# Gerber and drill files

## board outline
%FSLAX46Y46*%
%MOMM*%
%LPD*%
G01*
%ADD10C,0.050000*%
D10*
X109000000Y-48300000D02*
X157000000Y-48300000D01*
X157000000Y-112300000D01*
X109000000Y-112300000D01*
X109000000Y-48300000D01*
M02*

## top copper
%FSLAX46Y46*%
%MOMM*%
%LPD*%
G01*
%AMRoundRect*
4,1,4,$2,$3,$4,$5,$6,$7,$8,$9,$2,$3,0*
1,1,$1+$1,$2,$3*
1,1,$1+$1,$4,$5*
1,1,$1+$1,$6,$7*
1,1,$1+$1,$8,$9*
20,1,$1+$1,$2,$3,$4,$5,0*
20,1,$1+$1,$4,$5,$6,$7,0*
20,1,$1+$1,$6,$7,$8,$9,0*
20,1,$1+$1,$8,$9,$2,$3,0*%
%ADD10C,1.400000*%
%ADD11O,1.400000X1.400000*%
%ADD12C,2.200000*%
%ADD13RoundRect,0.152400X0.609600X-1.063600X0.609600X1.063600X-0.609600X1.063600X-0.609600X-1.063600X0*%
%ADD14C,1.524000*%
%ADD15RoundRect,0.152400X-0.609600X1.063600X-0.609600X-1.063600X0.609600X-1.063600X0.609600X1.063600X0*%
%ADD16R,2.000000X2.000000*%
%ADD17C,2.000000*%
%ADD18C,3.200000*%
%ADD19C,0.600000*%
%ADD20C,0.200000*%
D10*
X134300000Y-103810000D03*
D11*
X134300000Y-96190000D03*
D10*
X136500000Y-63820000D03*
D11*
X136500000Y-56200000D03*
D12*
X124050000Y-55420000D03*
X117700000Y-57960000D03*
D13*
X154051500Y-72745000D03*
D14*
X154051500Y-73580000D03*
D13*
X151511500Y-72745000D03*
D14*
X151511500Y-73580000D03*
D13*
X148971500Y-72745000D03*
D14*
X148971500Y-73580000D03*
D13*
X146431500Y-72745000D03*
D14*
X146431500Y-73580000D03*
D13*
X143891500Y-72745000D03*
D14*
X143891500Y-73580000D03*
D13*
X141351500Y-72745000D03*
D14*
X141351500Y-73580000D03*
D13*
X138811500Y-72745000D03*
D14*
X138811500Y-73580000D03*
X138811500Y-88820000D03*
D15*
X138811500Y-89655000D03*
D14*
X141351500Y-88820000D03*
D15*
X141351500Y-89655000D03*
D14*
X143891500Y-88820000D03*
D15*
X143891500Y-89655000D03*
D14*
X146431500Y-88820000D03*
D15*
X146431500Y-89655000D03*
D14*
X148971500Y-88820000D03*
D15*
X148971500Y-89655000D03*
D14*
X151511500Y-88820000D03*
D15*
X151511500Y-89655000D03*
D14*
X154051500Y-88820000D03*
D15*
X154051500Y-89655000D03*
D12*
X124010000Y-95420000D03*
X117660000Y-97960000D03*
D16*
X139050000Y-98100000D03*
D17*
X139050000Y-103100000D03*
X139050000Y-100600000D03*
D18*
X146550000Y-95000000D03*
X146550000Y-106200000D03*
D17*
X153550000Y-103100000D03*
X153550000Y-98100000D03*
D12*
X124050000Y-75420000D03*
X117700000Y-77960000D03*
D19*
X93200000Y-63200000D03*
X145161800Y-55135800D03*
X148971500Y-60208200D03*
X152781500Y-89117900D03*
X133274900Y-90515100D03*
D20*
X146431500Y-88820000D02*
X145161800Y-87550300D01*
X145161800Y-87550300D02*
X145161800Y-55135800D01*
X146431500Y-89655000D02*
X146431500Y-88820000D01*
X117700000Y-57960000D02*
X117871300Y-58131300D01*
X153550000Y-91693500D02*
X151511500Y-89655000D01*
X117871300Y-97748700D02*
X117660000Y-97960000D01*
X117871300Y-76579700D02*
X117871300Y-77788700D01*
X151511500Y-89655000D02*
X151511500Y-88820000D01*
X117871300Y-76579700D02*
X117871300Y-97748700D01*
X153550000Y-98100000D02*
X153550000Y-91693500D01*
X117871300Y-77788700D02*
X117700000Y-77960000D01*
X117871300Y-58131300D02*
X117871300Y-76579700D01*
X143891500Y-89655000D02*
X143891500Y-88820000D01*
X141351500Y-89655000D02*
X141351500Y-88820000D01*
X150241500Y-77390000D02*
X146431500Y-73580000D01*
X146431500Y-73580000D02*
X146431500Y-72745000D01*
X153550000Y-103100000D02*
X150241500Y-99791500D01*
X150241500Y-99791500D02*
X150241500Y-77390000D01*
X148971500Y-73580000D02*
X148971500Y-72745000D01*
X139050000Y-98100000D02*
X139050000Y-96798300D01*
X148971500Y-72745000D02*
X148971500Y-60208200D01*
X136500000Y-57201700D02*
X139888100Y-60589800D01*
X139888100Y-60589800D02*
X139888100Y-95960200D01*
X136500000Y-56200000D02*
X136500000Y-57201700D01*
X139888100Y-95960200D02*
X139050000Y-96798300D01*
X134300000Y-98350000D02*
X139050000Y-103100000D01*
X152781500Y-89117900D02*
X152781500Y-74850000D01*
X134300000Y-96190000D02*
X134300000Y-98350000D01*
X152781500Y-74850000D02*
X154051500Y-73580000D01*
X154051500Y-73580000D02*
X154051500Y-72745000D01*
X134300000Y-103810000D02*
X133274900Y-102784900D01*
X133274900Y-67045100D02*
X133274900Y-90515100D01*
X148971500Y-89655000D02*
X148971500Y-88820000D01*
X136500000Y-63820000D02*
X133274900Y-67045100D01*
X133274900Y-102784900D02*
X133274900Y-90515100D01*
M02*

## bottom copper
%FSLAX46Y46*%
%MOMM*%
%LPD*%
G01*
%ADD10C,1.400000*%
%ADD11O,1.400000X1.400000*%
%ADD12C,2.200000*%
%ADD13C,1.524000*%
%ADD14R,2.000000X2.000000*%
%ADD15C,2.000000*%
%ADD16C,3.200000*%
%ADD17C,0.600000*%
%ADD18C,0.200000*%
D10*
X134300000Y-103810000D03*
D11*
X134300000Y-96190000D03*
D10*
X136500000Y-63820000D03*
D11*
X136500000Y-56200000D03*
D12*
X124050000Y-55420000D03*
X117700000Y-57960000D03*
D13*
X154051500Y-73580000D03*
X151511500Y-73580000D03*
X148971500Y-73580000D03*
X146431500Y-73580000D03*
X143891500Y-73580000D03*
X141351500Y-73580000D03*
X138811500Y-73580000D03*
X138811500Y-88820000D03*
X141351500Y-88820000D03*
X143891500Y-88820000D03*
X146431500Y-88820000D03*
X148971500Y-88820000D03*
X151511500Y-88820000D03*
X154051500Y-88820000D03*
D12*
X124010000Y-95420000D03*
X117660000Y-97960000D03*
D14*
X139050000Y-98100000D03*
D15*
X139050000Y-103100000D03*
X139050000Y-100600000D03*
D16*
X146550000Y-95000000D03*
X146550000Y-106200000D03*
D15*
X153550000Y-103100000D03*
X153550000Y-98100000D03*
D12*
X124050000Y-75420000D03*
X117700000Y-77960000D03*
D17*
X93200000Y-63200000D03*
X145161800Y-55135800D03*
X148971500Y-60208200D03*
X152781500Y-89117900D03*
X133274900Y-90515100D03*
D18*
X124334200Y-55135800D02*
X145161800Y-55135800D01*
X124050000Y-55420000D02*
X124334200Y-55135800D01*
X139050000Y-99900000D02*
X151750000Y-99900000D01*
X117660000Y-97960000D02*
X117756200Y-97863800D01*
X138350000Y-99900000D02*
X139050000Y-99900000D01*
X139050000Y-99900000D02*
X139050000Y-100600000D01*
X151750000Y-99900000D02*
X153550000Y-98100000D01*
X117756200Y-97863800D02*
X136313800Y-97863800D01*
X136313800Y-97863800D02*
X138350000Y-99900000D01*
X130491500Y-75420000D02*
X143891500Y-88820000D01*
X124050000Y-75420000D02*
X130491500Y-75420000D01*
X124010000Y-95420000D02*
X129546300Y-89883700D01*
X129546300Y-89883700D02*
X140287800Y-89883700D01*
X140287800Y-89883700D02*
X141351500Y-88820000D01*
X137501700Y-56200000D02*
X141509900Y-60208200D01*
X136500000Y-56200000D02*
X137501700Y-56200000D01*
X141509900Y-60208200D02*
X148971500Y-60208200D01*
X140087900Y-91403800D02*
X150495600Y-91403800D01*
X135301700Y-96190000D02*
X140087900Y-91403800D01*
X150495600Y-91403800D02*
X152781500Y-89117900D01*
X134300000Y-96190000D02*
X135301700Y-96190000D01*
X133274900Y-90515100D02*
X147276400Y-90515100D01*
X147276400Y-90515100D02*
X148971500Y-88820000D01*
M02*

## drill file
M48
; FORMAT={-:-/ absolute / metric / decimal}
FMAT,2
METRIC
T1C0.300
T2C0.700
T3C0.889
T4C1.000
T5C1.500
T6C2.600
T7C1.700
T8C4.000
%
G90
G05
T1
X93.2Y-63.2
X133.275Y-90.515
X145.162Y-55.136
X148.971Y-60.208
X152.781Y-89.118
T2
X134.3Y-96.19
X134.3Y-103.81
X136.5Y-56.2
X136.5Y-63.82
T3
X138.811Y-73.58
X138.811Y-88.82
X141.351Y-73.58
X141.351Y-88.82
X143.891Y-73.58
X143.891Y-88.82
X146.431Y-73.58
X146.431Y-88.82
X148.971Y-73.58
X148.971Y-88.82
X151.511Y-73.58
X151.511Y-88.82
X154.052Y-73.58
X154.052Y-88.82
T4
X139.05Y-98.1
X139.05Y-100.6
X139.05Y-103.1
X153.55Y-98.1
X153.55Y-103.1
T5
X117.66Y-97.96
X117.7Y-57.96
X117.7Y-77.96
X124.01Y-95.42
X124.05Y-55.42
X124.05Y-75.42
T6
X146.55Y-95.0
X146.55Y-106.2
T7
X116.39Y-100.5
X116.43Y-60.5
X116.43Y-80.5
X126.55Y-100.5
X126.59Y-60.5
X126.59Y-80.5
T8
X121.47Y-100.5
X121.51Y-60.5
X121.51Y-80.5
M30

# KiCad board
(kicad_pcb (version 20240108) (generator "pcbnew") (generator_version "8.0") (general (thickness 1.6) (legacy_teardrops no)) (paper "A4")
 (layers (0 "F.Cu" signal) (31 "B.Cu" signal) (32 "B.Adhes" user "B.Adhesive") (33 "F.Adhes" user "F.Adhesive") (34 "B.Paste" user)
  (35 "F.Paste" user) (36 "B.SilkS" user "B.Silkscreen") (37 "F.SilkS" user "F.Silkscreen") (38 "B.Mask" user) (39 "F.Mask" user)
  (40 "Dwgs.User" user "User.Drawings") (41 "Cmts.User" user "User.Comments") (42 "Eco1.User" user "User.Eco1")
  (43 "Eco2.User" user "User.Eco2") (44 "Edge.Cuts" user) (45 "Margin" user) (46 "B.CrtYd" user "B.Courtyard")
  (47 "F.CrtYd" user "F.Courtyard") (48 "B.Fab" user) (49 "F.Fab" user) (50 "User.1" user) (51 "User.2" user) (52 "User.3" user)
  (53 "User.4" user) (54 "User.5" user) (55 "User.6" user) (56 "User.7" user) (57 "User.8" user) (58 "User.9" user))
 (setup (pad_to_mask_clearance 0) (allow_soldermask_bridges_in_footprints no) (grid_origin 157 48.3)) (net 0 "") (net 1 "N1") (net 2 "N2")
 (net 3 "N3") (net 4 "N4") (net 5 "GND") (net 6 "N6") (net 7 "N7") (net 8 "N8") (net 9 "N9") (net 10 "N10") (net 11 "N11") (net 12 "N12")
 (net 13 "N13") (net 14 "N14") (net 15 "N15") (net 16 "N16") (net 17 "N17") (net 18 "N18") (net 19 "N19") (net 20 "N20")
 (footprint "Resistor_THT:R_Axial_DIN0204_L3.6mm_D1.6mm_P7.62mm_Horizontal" (layer "F.Cu") (at 134.3 103.81 90)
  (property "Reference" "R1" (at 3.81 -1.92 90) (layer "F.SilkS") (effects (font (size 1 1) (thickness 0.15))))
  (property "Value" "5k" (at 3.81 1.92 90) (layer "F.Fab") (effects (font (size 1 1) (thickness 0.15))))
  (pad "1" thru_hole circle (at 0 0 90) (size 1.4 1.4) (drill 0.7) (layers "*.Cu" "*.Mask") (remove_unused_layers no) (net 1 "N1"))
  (pad "2" thru_hole oval (at 7.62 0 90) (size 1.4 1.4) (drill 0.7) (layers "*.Cu" "*.Mask") (remove_unused_layers no) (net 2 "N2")))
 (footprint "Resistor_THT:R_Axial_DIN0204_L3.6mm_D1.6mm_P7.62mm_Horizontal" (layer "F.Cu") (at 136.5 63.82 90)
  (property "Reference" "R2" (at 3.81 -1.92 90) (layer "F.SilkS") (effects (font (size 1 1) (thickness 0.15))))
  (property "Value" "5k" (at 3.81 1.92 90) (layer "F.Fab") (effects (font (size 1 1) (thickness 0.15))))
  (pad "1" thru_hole circle (at 0 0 90) (size 1.4 1.4) (drill 0.7) (layers "*.Cu" "*.Mask") (remove_unused_layers no) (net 1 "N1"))
  (pad "2" thru_hole oval (at 7.62 0 90) (size 1.4 1.4) (drill 0.7) (layers "*.Cu" "*.Mask") (remove_unused_layers no) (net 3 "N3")))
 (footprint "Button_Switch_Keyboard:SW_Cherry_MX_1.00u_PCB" (layer "F.Cu") (at 124.05 55.42)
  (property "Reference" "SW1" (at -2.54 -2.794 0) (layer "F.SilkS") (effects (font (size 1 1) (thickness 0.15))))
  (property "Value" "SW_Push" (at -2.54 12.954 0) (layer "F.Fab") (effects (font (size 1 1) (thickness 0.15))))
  (pad "" np_thru_hole circle (at -7.62 5.08) (size 1.7 1.7) (drill 1.7) (layers "*.Cu" "*.Mask"))
  (pad "" np_thru_hole circle (at -2.54 5.08) (size 4 4) (drill 4) (layers "*.Cu" "*.Mask"))
  (pad "" np_thru_hole circle (at 2.54 5.08) (size 1.7 1.7) (drill 1.7) (layers "*.Cu" "*.Mask"))
  (pad "1" thru_hole circle (at 0 0) (size 2.2 2.2) (drill 1.5) (layers "*.Cu" "*.Mask") (remove_unused_layers no) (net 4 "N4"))
  (pad "2" thru_hole circle (at -6.35 2.54) (size 2.2 2.2) (drill 1.5) (layers "*.Cu" "*.Mask") (remove_unused_layers no) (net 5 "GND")))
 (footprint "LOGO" (layer "F.Cu") (at 148.920677 59.275013 -90)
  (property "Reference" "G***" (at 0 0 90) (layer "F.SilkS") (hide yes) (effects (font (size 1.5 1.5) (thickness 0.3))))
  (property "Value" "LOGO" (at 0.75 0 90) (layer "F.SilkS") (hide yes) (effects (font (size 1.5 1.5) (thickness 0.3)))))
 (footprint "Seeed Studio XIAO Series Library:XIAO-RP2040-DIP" (layer "F.Cu") (at 146.4315 81.2 -90)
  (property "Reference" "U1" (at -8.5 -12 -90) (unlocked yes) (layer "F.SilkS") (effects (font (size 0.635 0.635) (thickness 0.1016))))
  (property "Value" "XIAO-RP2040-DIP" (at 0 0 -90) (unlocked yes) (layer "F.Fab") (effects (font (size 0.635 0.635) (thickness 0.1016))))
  (pad "1" smd roundrect (at -8.455 -7.62 90) (size 2.432 1.524) (layers "F.Cu" "F.Mask") (roundrect_rratio 0.1) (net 2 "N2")
   (thermal_bridge_angle 45))
  (pad "1" thru_hole circle (at -7.62 -7.62 90) (size 1.524 1.524) (drill 0.889) (layers "*.Cu" "*.Mask") (remove_unused_layers no)
   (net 2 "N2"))
  (pad "2" smd roundrect (at -8.455 -5.08 90) (size 2.432 1.524) (layers "F.Cu" "F.Mask") (roundrect_rratio 0.1) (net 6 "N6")
   (thermal_bridge_angle 45))
  (pad "2" thru_hole circle (at -7.62 -5.08 90) (size 1.524 1.524) (drill 0.889) (layers "*.Cu" "*.Mask") (remove_unused_layers no)
   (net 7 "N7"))
  (pad "3" smd roundrect (at -8.455 -2.54 90) (size 2.432 1.524) (layers "F.Cu" "F.Mask") (roundrect_rratio 0.1) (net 3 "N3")
   (thermal_bridge_angle 45))
  (pad "3" thru_hole circle (at -7.62 -2.54 90) (size 1.524 1.524) (drill 0.889) (layers "*.Cu" "*.Mask") (remove_unused_layers no)
   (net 3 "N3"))
  (pad "4" smd roundrect (at -8.455 0 90) (size 2.432 1.524) (layers "F.Cu" "F.Mask") (roundrect_rratio 0.1) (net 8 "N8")
   (thermal_bridge_angle 45))
  (pad "4" thru_hole circle (at -7.62 0 90) (size 1.524 1.524) (drill 0.889) (layers "*.Cu" "*.Mask") (remove_unused_layers no) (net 8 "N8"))
  (pad "5" smd roundrect (at -8.455 2.54 90) (size 2.432 1.524) (layers "F.Cu" "F.Mask") (roundrect_rratio 0.1) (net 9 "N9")
   (thermal_bridge_angle 45))
  (pad "5" thru_hole circle (at -7.62 2.54 90) (size 1.524 1.524) (drill 0.889) (layers "*.Cu" "*.Mask") (remove_unused_layers no)
   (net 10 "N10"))
  (pad "6" smd roundrect (at -8.455 5.08 90) (size 2.432 1.524) (layers "F.Cu" "F.Mask") (roundrect_rratio 0.1) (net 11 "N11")
   (thermal_bridge_angle 45))
  (pad "6" thru_hole circle (at -7.62 5.08 90) (size 1.524 1.524) (drill 0.889) (layers "*.Cu" "*.Mask") (remove_unused_layers no)
   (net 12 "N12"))
  (pad "7" smd roundrect (at -8.455 7.62 90) (size 2.432 1.524) (layers "F.Cu" "F.Mask") (roundrect_rratio 0.1) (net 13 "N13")
   (thermal_bridge_angle 45))
  (pad "7" thru_hole circle (at -7.62 7.62 90) (size 1.524 1.524) (drill 0.889) (layers "*.Cu" "*.Mask") (remove_unused_layers no)
   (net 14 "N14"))
  (pad "8" thru_hole circle (at 7.62 7.62 270) (size 1.524 1.524) (drill 0.889) (layers "*.Cu" "*.Mask") (remove_unused_layers no)
   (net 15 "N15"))
  (pad "8" smd roundrect (at 8.455 7.62 270) (size 2.432 1.524) (layers "F.Cu" "F.Mask") (roundrect_rratio 0.1) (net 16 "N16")
   (thermal_bridge_angle 45))
  (pad "9" thru_hole circle (at 7.62 5.08 270) (size 1.524 1.524) (drill 0.889) (layers "*.Cu" "*.Mask") (remove_unused_layers no)
   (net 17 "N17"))
  (pad "9" smd roundrect (at 8.455 5.08 270) (size 2.432 1.524) (layers "F.Cu" "F.Mask") (roundrect_rratio 0.1) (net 17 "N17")
   (thermal_bridge_angle 45))
  (pad "10" thru_hole circle (at 7.62 2.54 270) (size 1.524 1.524) (drill 0.889) (layers "*.Cu" "*.Mask") (remove_unused_layers no)
   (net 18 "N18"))
  (pad "10" smd roundrect (at 8.455 2.54 270) (size 2.432 1.524) (layers "F.Cu" "F.Mask") (roundrect_rratio 0.1) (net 18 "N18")
   (thermal_bridge_angle 45))
  (pad "11" thru_hole circle (at 7.62 0 270) (size 1.524 1.524) (drill 0.889) (layers "*.Cu" "*.Mask") (remove_unused_layers no)
   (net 4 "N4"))
  (pad "11" smd roundrect (at 8.455 0 270) (size 2.432 1.524) (layers "F.Cu" "F.Mask") (roundrect_rratio 0.1) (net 4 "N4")
   (thermal_bridge_angle 45))
  (pad "12" thru_hole circle (at 7.62 -2.54 270) (size 1.524 1.524) (drill 0.889) (layers "*.Cu" "*.Mask") (remove_unused_layers no)
   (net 1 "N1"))
  (pad "12" smd roundrect (at 8.455 -2.54 270) (size 2.432 1.524) (layers "F.Cu" "F.Mask") (roundrect_rratio 0.1) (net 1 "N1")
   (thermal_bridge_angle 45))
  (pad "13" thru_hole circle (at 7.62 -5.08 270) (size 1.524 1.524) (drill 0.889) (layers "*.Cu" "*.Mask") (remove_unused_layers no)
   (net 5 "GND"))
  (pad "13" smd roundrect (at 8.455 -5.08 270) (size 2.432 1.524) (layers "F.Cu" "F.Mask") (roundrect_rratio 0.1) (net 5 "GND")
   (thermal_bridge_angle 45))
  (pad "14" thru_hole circle (at 7.62 -7.62 270) (size 1.524 1.524) (drill 0.889) (layers "*.Cu" "*.Mask") (remove_unused_layers no)
   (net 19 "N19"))
  (pad "14" smd roundrect (at 8.455 -7.62 270) (size 2.432 1.524) (layers "F.Cu" "F.Mask") (roundrect_rratio 0.1) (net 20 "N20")
   (thermal_bridge_angle 45)))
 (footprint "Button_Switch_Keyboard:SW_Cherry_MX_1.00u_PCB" (layer "F.Cu") (at 124.01 95.42)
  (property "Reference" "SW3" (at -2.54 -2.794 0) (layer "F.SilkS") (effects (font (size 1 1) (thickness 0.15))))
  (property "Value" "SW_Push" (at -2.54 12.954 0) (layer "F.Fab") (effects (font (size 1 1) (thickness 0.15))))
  (pad "" np_thru_hole circle (at -7.62 5.08) (size 1.7 1.7) (drill 1.7) (layers "*.Cu" "*.Mask"))
  (pad "" np_thru_hole circle (at -2.54 5.08) (size 4 4) (drill 4) (layers "*.Cu" "*.Mask"))
  (pad "" np_thru_hole circle (at 2.54 5.08) (size 1.7 1.7) (drill 1.7) (layers "*.Cu" "*.Mask"))
  (pad "1" thru_hole circle (at 0 0) (size 2.2 2.2) (drill 1.5) (layers "*.Cu" "*.Mask") (remove_unused_layers no) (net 17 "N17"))
  (pad "2" thru_hole circle (at -6.35 2.54) (size 2.2 2.2) (drill 1.5) (layers "*.Cu" "*.Mask") (remove_unused_layers no) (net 5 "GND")))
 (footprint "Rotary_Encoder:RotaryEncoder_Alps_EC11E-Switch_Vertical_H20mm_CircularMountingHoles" (layer "F.Cu") (at 139.05 98.1)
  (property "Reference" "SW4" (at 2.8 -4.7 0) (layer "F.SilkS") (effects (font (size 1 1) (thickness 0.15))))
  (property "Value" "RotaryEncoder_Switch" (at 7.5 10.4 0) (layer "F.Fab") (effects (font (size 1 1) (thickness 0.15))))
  (pad "A" thru_hole rect (at 0 0) (size 2 2) (drill 1) (layers "*.Cu" "*.Mask") (remove_unused_layers no) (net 3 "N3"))
  (pad "B" thru_hole circle (at 0 5) (size 2 2) (drill 1) (layers "*.Cu" "*.Mask") (remove_unused_layers no) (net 2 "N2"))
  (pad "C" thru_hole circle (at 0 2.5) (size 2 2) (drill 1) (layers "*.Cu" "*.Mask") (remove_unused_layers no) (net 5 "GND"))
  (pad "MP" thru_hole circle (at 7.5 -3.1) (size 3.2 3.2) (drill 2.6) (layers "*.Cu" "*.Mask") (remove_unused_layers no))
  (pad "MP" thru_hole circle (at 7.5 8.1) (size 3.2 3.2) (drill 2.6) (layers "*.Cu" "*.Mask") (remove_unused_layers no))
  (pad "S1" thru_hole circle (at 14.5 5) (size 2 2) (drill 1) (layers "*.Cu" "*.Mask") (remove_unused_layers no) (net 8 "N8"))
  (pad "S2" thru_hole circle (at 14.5 0) (size 2 2) (drill 1) (layers "*.Cu" "*.Mask") (remove_unused_layers no) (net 5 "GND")))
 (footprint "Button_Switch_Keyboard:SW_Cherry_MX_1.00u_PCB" (layer "F.Cu") (at 124.05 75.42)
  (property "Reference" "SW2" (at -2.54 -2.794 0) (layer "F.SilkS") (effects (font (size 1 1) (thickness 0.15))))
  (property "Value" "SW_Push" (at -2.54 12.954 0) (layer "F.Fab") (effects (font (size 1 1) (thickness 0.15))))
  (pad "" np_thru_hole circle (at -7.62 5.08) (size 1.7 1.7) (drill 1.7) (layers "*.Cu" "*.Mask"))
  (pad "" np_thru_hole circle (at -2.54 5.08) (size 4 4) (drill 4) (layers "*.Cu" "*.Mask"))
  (pad "" np_thru_hole circle (at 2.54 5.08) (size 1.7 1.7) (drill 1.7) (layers "*.Cu" "*.Mask"))
  (pad "1" thru_hole circle (at 0 0) (size 2.2 2.2) (drill 1.5) (layers "*.Cu" "*.Mask") (remove_unused_layers no) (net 18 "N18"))
  (pad "2" thru_hole circle (at -6.35 2.54) (size 2.2 2.2) (drill 1.5) (layers "*.Cu" "*.Mask") (remove_unused_layers no) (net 5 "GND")))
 (gr_rect (start 109 48.3) (end 157 112.3) (stroke (width 0.05) (type default)) (fill none) (layer "Edge.Cuts"))
 (via (at 93.2 63.2) (size 0.6) (drill 0.3) (layers "F.Cu" "B.Cu") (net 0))
 (segment (start 146.4315 88.82) (end 145.1618 87.5503) (width 0.2) (layer "F.Cu") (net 4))
 (segment (start 145.1618 87.5503) (end 145.1618 55.1358) (width 0.2) (layer "F.Cu") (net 4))
 (segment (start 146.4315 89.655) (end 146.4315 88.82) (width 0.2) (layer "F.Cu") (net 4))
 (via (at 145.1618 55.1358) (size 0.6) (drill 0.3) (layers "F.Cu" "B.Cu") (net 4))
 (segment (start 124.3342 55.1358) (end 145.1618 55.1358) (width 0.2) (layer "B.Cu") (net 4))
 (segment (start 124.05 55.42) (end 124.3342 55.1358) (width 0.2) (layer "B.Cu") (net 4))
 (segment (start 117.7 57.96) (end 117.8713 58.1313) (width 0.2) (layer "F.Cu") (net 5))
 (segment (start 153.55 91.6935) (end 151.5115 89.655) (width 0.2) (layer "F.Cu") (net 5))
 (segment (start 117.8713 97.7487) (end 117.66 97.96) (width 0.2) (layer "F.Cu") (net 5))
 (segment (start 117.8713 76.5797) (end 117.8713 77.7887) (width 0.2) (layer "F.Cu") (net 5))
 (segment (start 151.5115 89.655) (end 151.5115 88.82) (width 0.2) (layer "F.Cu") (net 5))
 (segment (start 117.8713 76.5797) (end 117.8713 97.7487) (width 0.2) (layer "F.Cu") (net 5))
 (segment (start 153.55 98.1) (end 153.55 91.6935) (width 0.2) (layer "F.Cu") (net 5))
 (segment (start 117.8713 77.7887) (end 117.7 77.96) (width 0.2) (layer "F.Cu") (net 5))
 (segment (start 117.8713 58.1313) (end 117.8713 76.5797) (width 0.2) (layer "F.Cu") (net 5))
 (segment (start 139.05 99.9) (end 151.75 99.9) (width 0.2) (layer "B.Cu") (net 5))
 (segment (start 117.66 97.96) (end 117.7562 97.8638) (width 0.2) (layer "B.Cu") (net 5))
 (segment (start 138.35 99.9) (end 139.05 99.9) (width 0.2) (layer "B.Cu") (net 5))
 (segment (start 139.05 99.9) (end 139.05 100.6) (width 0.2) (layer "B.Cu") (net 5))
 (segment (start 151.75 99.9) (end 153.55 98.1) (width 0.2) (layer "B.Cu") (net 5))
 (segment (start 117.7562 97.8638) (end 136.3138 97.8638) (width 0.2) (layer "B.Cu") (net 5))
 (segment (start 136.3138 97.8638) (end 138.35 99.9) (width 0.2) (layer "B.Cu") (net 5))
 (segment (start 143.8915 89.655) (end 143.8915 88.82) (width 0.2) (layer "F.Cu") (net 18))
 (segment (start 130.4915 75.42) (end 143.8915 88.82) (width 0.2) (layer "B.Cu") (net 18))
 (segment (start 124.05 75.42) (end 130.4915 75.42) (width 0.2) (layer "B.Cu") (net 18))
 (segment (start 141.3515 89.655) (end 141.3515 88.82) (width 0.2) (layer "F.Cu") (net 17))
 (segment (start 124.01 95.42) (end 129.5463 89.8837) (width 0.2) (layer "B.Cu") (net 17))
 (segment (start 129.5463 89.8837) (end 140.2878 89.8837) (width 0.2) (layer "B.Cu") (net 17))
 (segment (start 140.2878 89.8837) (end 141.3515 88.82) (width 0.2) (layer "B.Cu") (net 17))
 (segment (start 150.2415 77.39) (end 146.4315 73.58) (width 0.2) (layer "F.Cu") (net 8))
 (segment (start 146.4315 73.58) (end 146.4315 72.745) (width 0.2) (layer "F.Cu") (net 8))
 (segment (start 153.55 103.1) (end 150.2415 99.7915) (width 0.2) (layer "F.Cu") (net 8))
 (segment (start 150.2415 99.7915) (end 150.2415 77.39) (width 0.2) (layer "F.Cu") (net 8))
 (segment (start 148.9715 73.58) (end 148.9715 72.745) (width 0.2) (layer "F.Cu") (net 3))
 (segment (start 139.05 98.1) (end 139.05 96.7983) (width 0.2) (layer "F.Cu") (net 3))
 (segment (start 148.9715 72.745) (end 148.9715 60.2082) (width 0.2) (layer "F.Cu") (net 3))
 (segment (start 136.5 57.2017) (end 139.8881 60.5898) (width 0.2) (layer "F.Cu") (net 3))
 (segment (start 139.8881 60.5898) (end 139.8881 95.9602) (width 0.2) (layer "F.Cu") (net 3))
 (segment (start 136.5 56.2) (end 136.5 57.2017) (width 0.2) (layer "F.Cu") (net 3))
 (segment (start 139.8881 95.9602) (end 139.05 96.7983) (width 0.2) (layer "F.Cu") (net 3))
 (via (at 148.9715 60.2082) (size 0.6) (drill 0.3) (layers "F.Cu" "B.Cu") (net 3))
 (segment (start 137.5017 56.2) (end 141.5099 60.2082) (width 0.2) (layer "B.Cu") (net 3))
 (segment (start 136.5 56.2) (end 137.5017 56.2) (width 0.2) (layer "B.Cu") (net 3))
 (segment (start 141.5099 60.2082) (end 148.9715 60.2082) (width 0.2) (layer "B.Cu") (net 3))
 (segment (start 134.3 98.35) (end 139.05 103.1) (width 0.2) (layer "F.Cu") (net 2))
 (segment (start 152.7815 89.1179) (end 152.7815 74.85) (width 0.2) (layer "F.Cu") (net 2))
 (segment (start 134.3 96.19) (end 134.3 98.35) (width 0.2) (layer "F.Cu") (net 2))
 (segment (start 152.7815 74.85) (end 154.0515 73.58) (width 0.2) (layer "F.Cu") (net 2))
 (segment (start 154.0515 73.58) (end 154.0515 72.745) (width 0.2) (layer "F.Cu") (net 2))
 (via (at 152.7815 89.1179) (size 0.6) (drill 0.3) (layers "F.Cu" "B.Cu") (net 2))
 (segment (start 140.0879 91.4038) (end 150.4956 91.4038) (width 0.2) (layer "B.Cu") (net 2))
 (segment (start 135.3017 96.19) (end 140.0879 91.4038) (width 0.2) (layer "B.Cu") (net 2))
 (segment (start 150.4956 91.4038) (end 152.7815 89.1179) (width 0.2) (layer "B.Cu") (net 2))
 (segment (start 134.3 96.19) (end 135.3017 96.19) (width 0.2) (layer "B.Cu") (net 2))
 (segment (start 134.3 103.81) (end 133.2749 102.7849) (width 0.2) (layer "F.Cu") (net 1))
 (segment (start 133.2749 67.0451) (end 133.2749 90.5151) (width 0.2) (layer "F.Cu") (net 1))
 (segment (start 148.9715 89.655) (end 148.9715 88.82) (width 0.2) (layer "F.Cu") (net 1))
 (segment (start 136.5 63.82) (end 133.2749 67.0451) (width 0.2) (layer "F.Cu") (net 1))
 (segment (start 133.2749 102.7849) (end 133.2749 90.5151) (width 0.2) (layer "F.Cu") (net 1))
 (via (at 133.2749 90.5151) (size 0.6) (drill 0.3) (layers "F.Cu" "B.Cu") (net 1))
 (segment (start 133.2749 90.5151) (end 147.2764 90.5151) (width 0.2) (layer "B.Cu") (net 1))
 (segment (start 147.2764 90.5151) (end 148.9715 88.82) (width 0.2) (layer "B.Cu") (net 1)))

